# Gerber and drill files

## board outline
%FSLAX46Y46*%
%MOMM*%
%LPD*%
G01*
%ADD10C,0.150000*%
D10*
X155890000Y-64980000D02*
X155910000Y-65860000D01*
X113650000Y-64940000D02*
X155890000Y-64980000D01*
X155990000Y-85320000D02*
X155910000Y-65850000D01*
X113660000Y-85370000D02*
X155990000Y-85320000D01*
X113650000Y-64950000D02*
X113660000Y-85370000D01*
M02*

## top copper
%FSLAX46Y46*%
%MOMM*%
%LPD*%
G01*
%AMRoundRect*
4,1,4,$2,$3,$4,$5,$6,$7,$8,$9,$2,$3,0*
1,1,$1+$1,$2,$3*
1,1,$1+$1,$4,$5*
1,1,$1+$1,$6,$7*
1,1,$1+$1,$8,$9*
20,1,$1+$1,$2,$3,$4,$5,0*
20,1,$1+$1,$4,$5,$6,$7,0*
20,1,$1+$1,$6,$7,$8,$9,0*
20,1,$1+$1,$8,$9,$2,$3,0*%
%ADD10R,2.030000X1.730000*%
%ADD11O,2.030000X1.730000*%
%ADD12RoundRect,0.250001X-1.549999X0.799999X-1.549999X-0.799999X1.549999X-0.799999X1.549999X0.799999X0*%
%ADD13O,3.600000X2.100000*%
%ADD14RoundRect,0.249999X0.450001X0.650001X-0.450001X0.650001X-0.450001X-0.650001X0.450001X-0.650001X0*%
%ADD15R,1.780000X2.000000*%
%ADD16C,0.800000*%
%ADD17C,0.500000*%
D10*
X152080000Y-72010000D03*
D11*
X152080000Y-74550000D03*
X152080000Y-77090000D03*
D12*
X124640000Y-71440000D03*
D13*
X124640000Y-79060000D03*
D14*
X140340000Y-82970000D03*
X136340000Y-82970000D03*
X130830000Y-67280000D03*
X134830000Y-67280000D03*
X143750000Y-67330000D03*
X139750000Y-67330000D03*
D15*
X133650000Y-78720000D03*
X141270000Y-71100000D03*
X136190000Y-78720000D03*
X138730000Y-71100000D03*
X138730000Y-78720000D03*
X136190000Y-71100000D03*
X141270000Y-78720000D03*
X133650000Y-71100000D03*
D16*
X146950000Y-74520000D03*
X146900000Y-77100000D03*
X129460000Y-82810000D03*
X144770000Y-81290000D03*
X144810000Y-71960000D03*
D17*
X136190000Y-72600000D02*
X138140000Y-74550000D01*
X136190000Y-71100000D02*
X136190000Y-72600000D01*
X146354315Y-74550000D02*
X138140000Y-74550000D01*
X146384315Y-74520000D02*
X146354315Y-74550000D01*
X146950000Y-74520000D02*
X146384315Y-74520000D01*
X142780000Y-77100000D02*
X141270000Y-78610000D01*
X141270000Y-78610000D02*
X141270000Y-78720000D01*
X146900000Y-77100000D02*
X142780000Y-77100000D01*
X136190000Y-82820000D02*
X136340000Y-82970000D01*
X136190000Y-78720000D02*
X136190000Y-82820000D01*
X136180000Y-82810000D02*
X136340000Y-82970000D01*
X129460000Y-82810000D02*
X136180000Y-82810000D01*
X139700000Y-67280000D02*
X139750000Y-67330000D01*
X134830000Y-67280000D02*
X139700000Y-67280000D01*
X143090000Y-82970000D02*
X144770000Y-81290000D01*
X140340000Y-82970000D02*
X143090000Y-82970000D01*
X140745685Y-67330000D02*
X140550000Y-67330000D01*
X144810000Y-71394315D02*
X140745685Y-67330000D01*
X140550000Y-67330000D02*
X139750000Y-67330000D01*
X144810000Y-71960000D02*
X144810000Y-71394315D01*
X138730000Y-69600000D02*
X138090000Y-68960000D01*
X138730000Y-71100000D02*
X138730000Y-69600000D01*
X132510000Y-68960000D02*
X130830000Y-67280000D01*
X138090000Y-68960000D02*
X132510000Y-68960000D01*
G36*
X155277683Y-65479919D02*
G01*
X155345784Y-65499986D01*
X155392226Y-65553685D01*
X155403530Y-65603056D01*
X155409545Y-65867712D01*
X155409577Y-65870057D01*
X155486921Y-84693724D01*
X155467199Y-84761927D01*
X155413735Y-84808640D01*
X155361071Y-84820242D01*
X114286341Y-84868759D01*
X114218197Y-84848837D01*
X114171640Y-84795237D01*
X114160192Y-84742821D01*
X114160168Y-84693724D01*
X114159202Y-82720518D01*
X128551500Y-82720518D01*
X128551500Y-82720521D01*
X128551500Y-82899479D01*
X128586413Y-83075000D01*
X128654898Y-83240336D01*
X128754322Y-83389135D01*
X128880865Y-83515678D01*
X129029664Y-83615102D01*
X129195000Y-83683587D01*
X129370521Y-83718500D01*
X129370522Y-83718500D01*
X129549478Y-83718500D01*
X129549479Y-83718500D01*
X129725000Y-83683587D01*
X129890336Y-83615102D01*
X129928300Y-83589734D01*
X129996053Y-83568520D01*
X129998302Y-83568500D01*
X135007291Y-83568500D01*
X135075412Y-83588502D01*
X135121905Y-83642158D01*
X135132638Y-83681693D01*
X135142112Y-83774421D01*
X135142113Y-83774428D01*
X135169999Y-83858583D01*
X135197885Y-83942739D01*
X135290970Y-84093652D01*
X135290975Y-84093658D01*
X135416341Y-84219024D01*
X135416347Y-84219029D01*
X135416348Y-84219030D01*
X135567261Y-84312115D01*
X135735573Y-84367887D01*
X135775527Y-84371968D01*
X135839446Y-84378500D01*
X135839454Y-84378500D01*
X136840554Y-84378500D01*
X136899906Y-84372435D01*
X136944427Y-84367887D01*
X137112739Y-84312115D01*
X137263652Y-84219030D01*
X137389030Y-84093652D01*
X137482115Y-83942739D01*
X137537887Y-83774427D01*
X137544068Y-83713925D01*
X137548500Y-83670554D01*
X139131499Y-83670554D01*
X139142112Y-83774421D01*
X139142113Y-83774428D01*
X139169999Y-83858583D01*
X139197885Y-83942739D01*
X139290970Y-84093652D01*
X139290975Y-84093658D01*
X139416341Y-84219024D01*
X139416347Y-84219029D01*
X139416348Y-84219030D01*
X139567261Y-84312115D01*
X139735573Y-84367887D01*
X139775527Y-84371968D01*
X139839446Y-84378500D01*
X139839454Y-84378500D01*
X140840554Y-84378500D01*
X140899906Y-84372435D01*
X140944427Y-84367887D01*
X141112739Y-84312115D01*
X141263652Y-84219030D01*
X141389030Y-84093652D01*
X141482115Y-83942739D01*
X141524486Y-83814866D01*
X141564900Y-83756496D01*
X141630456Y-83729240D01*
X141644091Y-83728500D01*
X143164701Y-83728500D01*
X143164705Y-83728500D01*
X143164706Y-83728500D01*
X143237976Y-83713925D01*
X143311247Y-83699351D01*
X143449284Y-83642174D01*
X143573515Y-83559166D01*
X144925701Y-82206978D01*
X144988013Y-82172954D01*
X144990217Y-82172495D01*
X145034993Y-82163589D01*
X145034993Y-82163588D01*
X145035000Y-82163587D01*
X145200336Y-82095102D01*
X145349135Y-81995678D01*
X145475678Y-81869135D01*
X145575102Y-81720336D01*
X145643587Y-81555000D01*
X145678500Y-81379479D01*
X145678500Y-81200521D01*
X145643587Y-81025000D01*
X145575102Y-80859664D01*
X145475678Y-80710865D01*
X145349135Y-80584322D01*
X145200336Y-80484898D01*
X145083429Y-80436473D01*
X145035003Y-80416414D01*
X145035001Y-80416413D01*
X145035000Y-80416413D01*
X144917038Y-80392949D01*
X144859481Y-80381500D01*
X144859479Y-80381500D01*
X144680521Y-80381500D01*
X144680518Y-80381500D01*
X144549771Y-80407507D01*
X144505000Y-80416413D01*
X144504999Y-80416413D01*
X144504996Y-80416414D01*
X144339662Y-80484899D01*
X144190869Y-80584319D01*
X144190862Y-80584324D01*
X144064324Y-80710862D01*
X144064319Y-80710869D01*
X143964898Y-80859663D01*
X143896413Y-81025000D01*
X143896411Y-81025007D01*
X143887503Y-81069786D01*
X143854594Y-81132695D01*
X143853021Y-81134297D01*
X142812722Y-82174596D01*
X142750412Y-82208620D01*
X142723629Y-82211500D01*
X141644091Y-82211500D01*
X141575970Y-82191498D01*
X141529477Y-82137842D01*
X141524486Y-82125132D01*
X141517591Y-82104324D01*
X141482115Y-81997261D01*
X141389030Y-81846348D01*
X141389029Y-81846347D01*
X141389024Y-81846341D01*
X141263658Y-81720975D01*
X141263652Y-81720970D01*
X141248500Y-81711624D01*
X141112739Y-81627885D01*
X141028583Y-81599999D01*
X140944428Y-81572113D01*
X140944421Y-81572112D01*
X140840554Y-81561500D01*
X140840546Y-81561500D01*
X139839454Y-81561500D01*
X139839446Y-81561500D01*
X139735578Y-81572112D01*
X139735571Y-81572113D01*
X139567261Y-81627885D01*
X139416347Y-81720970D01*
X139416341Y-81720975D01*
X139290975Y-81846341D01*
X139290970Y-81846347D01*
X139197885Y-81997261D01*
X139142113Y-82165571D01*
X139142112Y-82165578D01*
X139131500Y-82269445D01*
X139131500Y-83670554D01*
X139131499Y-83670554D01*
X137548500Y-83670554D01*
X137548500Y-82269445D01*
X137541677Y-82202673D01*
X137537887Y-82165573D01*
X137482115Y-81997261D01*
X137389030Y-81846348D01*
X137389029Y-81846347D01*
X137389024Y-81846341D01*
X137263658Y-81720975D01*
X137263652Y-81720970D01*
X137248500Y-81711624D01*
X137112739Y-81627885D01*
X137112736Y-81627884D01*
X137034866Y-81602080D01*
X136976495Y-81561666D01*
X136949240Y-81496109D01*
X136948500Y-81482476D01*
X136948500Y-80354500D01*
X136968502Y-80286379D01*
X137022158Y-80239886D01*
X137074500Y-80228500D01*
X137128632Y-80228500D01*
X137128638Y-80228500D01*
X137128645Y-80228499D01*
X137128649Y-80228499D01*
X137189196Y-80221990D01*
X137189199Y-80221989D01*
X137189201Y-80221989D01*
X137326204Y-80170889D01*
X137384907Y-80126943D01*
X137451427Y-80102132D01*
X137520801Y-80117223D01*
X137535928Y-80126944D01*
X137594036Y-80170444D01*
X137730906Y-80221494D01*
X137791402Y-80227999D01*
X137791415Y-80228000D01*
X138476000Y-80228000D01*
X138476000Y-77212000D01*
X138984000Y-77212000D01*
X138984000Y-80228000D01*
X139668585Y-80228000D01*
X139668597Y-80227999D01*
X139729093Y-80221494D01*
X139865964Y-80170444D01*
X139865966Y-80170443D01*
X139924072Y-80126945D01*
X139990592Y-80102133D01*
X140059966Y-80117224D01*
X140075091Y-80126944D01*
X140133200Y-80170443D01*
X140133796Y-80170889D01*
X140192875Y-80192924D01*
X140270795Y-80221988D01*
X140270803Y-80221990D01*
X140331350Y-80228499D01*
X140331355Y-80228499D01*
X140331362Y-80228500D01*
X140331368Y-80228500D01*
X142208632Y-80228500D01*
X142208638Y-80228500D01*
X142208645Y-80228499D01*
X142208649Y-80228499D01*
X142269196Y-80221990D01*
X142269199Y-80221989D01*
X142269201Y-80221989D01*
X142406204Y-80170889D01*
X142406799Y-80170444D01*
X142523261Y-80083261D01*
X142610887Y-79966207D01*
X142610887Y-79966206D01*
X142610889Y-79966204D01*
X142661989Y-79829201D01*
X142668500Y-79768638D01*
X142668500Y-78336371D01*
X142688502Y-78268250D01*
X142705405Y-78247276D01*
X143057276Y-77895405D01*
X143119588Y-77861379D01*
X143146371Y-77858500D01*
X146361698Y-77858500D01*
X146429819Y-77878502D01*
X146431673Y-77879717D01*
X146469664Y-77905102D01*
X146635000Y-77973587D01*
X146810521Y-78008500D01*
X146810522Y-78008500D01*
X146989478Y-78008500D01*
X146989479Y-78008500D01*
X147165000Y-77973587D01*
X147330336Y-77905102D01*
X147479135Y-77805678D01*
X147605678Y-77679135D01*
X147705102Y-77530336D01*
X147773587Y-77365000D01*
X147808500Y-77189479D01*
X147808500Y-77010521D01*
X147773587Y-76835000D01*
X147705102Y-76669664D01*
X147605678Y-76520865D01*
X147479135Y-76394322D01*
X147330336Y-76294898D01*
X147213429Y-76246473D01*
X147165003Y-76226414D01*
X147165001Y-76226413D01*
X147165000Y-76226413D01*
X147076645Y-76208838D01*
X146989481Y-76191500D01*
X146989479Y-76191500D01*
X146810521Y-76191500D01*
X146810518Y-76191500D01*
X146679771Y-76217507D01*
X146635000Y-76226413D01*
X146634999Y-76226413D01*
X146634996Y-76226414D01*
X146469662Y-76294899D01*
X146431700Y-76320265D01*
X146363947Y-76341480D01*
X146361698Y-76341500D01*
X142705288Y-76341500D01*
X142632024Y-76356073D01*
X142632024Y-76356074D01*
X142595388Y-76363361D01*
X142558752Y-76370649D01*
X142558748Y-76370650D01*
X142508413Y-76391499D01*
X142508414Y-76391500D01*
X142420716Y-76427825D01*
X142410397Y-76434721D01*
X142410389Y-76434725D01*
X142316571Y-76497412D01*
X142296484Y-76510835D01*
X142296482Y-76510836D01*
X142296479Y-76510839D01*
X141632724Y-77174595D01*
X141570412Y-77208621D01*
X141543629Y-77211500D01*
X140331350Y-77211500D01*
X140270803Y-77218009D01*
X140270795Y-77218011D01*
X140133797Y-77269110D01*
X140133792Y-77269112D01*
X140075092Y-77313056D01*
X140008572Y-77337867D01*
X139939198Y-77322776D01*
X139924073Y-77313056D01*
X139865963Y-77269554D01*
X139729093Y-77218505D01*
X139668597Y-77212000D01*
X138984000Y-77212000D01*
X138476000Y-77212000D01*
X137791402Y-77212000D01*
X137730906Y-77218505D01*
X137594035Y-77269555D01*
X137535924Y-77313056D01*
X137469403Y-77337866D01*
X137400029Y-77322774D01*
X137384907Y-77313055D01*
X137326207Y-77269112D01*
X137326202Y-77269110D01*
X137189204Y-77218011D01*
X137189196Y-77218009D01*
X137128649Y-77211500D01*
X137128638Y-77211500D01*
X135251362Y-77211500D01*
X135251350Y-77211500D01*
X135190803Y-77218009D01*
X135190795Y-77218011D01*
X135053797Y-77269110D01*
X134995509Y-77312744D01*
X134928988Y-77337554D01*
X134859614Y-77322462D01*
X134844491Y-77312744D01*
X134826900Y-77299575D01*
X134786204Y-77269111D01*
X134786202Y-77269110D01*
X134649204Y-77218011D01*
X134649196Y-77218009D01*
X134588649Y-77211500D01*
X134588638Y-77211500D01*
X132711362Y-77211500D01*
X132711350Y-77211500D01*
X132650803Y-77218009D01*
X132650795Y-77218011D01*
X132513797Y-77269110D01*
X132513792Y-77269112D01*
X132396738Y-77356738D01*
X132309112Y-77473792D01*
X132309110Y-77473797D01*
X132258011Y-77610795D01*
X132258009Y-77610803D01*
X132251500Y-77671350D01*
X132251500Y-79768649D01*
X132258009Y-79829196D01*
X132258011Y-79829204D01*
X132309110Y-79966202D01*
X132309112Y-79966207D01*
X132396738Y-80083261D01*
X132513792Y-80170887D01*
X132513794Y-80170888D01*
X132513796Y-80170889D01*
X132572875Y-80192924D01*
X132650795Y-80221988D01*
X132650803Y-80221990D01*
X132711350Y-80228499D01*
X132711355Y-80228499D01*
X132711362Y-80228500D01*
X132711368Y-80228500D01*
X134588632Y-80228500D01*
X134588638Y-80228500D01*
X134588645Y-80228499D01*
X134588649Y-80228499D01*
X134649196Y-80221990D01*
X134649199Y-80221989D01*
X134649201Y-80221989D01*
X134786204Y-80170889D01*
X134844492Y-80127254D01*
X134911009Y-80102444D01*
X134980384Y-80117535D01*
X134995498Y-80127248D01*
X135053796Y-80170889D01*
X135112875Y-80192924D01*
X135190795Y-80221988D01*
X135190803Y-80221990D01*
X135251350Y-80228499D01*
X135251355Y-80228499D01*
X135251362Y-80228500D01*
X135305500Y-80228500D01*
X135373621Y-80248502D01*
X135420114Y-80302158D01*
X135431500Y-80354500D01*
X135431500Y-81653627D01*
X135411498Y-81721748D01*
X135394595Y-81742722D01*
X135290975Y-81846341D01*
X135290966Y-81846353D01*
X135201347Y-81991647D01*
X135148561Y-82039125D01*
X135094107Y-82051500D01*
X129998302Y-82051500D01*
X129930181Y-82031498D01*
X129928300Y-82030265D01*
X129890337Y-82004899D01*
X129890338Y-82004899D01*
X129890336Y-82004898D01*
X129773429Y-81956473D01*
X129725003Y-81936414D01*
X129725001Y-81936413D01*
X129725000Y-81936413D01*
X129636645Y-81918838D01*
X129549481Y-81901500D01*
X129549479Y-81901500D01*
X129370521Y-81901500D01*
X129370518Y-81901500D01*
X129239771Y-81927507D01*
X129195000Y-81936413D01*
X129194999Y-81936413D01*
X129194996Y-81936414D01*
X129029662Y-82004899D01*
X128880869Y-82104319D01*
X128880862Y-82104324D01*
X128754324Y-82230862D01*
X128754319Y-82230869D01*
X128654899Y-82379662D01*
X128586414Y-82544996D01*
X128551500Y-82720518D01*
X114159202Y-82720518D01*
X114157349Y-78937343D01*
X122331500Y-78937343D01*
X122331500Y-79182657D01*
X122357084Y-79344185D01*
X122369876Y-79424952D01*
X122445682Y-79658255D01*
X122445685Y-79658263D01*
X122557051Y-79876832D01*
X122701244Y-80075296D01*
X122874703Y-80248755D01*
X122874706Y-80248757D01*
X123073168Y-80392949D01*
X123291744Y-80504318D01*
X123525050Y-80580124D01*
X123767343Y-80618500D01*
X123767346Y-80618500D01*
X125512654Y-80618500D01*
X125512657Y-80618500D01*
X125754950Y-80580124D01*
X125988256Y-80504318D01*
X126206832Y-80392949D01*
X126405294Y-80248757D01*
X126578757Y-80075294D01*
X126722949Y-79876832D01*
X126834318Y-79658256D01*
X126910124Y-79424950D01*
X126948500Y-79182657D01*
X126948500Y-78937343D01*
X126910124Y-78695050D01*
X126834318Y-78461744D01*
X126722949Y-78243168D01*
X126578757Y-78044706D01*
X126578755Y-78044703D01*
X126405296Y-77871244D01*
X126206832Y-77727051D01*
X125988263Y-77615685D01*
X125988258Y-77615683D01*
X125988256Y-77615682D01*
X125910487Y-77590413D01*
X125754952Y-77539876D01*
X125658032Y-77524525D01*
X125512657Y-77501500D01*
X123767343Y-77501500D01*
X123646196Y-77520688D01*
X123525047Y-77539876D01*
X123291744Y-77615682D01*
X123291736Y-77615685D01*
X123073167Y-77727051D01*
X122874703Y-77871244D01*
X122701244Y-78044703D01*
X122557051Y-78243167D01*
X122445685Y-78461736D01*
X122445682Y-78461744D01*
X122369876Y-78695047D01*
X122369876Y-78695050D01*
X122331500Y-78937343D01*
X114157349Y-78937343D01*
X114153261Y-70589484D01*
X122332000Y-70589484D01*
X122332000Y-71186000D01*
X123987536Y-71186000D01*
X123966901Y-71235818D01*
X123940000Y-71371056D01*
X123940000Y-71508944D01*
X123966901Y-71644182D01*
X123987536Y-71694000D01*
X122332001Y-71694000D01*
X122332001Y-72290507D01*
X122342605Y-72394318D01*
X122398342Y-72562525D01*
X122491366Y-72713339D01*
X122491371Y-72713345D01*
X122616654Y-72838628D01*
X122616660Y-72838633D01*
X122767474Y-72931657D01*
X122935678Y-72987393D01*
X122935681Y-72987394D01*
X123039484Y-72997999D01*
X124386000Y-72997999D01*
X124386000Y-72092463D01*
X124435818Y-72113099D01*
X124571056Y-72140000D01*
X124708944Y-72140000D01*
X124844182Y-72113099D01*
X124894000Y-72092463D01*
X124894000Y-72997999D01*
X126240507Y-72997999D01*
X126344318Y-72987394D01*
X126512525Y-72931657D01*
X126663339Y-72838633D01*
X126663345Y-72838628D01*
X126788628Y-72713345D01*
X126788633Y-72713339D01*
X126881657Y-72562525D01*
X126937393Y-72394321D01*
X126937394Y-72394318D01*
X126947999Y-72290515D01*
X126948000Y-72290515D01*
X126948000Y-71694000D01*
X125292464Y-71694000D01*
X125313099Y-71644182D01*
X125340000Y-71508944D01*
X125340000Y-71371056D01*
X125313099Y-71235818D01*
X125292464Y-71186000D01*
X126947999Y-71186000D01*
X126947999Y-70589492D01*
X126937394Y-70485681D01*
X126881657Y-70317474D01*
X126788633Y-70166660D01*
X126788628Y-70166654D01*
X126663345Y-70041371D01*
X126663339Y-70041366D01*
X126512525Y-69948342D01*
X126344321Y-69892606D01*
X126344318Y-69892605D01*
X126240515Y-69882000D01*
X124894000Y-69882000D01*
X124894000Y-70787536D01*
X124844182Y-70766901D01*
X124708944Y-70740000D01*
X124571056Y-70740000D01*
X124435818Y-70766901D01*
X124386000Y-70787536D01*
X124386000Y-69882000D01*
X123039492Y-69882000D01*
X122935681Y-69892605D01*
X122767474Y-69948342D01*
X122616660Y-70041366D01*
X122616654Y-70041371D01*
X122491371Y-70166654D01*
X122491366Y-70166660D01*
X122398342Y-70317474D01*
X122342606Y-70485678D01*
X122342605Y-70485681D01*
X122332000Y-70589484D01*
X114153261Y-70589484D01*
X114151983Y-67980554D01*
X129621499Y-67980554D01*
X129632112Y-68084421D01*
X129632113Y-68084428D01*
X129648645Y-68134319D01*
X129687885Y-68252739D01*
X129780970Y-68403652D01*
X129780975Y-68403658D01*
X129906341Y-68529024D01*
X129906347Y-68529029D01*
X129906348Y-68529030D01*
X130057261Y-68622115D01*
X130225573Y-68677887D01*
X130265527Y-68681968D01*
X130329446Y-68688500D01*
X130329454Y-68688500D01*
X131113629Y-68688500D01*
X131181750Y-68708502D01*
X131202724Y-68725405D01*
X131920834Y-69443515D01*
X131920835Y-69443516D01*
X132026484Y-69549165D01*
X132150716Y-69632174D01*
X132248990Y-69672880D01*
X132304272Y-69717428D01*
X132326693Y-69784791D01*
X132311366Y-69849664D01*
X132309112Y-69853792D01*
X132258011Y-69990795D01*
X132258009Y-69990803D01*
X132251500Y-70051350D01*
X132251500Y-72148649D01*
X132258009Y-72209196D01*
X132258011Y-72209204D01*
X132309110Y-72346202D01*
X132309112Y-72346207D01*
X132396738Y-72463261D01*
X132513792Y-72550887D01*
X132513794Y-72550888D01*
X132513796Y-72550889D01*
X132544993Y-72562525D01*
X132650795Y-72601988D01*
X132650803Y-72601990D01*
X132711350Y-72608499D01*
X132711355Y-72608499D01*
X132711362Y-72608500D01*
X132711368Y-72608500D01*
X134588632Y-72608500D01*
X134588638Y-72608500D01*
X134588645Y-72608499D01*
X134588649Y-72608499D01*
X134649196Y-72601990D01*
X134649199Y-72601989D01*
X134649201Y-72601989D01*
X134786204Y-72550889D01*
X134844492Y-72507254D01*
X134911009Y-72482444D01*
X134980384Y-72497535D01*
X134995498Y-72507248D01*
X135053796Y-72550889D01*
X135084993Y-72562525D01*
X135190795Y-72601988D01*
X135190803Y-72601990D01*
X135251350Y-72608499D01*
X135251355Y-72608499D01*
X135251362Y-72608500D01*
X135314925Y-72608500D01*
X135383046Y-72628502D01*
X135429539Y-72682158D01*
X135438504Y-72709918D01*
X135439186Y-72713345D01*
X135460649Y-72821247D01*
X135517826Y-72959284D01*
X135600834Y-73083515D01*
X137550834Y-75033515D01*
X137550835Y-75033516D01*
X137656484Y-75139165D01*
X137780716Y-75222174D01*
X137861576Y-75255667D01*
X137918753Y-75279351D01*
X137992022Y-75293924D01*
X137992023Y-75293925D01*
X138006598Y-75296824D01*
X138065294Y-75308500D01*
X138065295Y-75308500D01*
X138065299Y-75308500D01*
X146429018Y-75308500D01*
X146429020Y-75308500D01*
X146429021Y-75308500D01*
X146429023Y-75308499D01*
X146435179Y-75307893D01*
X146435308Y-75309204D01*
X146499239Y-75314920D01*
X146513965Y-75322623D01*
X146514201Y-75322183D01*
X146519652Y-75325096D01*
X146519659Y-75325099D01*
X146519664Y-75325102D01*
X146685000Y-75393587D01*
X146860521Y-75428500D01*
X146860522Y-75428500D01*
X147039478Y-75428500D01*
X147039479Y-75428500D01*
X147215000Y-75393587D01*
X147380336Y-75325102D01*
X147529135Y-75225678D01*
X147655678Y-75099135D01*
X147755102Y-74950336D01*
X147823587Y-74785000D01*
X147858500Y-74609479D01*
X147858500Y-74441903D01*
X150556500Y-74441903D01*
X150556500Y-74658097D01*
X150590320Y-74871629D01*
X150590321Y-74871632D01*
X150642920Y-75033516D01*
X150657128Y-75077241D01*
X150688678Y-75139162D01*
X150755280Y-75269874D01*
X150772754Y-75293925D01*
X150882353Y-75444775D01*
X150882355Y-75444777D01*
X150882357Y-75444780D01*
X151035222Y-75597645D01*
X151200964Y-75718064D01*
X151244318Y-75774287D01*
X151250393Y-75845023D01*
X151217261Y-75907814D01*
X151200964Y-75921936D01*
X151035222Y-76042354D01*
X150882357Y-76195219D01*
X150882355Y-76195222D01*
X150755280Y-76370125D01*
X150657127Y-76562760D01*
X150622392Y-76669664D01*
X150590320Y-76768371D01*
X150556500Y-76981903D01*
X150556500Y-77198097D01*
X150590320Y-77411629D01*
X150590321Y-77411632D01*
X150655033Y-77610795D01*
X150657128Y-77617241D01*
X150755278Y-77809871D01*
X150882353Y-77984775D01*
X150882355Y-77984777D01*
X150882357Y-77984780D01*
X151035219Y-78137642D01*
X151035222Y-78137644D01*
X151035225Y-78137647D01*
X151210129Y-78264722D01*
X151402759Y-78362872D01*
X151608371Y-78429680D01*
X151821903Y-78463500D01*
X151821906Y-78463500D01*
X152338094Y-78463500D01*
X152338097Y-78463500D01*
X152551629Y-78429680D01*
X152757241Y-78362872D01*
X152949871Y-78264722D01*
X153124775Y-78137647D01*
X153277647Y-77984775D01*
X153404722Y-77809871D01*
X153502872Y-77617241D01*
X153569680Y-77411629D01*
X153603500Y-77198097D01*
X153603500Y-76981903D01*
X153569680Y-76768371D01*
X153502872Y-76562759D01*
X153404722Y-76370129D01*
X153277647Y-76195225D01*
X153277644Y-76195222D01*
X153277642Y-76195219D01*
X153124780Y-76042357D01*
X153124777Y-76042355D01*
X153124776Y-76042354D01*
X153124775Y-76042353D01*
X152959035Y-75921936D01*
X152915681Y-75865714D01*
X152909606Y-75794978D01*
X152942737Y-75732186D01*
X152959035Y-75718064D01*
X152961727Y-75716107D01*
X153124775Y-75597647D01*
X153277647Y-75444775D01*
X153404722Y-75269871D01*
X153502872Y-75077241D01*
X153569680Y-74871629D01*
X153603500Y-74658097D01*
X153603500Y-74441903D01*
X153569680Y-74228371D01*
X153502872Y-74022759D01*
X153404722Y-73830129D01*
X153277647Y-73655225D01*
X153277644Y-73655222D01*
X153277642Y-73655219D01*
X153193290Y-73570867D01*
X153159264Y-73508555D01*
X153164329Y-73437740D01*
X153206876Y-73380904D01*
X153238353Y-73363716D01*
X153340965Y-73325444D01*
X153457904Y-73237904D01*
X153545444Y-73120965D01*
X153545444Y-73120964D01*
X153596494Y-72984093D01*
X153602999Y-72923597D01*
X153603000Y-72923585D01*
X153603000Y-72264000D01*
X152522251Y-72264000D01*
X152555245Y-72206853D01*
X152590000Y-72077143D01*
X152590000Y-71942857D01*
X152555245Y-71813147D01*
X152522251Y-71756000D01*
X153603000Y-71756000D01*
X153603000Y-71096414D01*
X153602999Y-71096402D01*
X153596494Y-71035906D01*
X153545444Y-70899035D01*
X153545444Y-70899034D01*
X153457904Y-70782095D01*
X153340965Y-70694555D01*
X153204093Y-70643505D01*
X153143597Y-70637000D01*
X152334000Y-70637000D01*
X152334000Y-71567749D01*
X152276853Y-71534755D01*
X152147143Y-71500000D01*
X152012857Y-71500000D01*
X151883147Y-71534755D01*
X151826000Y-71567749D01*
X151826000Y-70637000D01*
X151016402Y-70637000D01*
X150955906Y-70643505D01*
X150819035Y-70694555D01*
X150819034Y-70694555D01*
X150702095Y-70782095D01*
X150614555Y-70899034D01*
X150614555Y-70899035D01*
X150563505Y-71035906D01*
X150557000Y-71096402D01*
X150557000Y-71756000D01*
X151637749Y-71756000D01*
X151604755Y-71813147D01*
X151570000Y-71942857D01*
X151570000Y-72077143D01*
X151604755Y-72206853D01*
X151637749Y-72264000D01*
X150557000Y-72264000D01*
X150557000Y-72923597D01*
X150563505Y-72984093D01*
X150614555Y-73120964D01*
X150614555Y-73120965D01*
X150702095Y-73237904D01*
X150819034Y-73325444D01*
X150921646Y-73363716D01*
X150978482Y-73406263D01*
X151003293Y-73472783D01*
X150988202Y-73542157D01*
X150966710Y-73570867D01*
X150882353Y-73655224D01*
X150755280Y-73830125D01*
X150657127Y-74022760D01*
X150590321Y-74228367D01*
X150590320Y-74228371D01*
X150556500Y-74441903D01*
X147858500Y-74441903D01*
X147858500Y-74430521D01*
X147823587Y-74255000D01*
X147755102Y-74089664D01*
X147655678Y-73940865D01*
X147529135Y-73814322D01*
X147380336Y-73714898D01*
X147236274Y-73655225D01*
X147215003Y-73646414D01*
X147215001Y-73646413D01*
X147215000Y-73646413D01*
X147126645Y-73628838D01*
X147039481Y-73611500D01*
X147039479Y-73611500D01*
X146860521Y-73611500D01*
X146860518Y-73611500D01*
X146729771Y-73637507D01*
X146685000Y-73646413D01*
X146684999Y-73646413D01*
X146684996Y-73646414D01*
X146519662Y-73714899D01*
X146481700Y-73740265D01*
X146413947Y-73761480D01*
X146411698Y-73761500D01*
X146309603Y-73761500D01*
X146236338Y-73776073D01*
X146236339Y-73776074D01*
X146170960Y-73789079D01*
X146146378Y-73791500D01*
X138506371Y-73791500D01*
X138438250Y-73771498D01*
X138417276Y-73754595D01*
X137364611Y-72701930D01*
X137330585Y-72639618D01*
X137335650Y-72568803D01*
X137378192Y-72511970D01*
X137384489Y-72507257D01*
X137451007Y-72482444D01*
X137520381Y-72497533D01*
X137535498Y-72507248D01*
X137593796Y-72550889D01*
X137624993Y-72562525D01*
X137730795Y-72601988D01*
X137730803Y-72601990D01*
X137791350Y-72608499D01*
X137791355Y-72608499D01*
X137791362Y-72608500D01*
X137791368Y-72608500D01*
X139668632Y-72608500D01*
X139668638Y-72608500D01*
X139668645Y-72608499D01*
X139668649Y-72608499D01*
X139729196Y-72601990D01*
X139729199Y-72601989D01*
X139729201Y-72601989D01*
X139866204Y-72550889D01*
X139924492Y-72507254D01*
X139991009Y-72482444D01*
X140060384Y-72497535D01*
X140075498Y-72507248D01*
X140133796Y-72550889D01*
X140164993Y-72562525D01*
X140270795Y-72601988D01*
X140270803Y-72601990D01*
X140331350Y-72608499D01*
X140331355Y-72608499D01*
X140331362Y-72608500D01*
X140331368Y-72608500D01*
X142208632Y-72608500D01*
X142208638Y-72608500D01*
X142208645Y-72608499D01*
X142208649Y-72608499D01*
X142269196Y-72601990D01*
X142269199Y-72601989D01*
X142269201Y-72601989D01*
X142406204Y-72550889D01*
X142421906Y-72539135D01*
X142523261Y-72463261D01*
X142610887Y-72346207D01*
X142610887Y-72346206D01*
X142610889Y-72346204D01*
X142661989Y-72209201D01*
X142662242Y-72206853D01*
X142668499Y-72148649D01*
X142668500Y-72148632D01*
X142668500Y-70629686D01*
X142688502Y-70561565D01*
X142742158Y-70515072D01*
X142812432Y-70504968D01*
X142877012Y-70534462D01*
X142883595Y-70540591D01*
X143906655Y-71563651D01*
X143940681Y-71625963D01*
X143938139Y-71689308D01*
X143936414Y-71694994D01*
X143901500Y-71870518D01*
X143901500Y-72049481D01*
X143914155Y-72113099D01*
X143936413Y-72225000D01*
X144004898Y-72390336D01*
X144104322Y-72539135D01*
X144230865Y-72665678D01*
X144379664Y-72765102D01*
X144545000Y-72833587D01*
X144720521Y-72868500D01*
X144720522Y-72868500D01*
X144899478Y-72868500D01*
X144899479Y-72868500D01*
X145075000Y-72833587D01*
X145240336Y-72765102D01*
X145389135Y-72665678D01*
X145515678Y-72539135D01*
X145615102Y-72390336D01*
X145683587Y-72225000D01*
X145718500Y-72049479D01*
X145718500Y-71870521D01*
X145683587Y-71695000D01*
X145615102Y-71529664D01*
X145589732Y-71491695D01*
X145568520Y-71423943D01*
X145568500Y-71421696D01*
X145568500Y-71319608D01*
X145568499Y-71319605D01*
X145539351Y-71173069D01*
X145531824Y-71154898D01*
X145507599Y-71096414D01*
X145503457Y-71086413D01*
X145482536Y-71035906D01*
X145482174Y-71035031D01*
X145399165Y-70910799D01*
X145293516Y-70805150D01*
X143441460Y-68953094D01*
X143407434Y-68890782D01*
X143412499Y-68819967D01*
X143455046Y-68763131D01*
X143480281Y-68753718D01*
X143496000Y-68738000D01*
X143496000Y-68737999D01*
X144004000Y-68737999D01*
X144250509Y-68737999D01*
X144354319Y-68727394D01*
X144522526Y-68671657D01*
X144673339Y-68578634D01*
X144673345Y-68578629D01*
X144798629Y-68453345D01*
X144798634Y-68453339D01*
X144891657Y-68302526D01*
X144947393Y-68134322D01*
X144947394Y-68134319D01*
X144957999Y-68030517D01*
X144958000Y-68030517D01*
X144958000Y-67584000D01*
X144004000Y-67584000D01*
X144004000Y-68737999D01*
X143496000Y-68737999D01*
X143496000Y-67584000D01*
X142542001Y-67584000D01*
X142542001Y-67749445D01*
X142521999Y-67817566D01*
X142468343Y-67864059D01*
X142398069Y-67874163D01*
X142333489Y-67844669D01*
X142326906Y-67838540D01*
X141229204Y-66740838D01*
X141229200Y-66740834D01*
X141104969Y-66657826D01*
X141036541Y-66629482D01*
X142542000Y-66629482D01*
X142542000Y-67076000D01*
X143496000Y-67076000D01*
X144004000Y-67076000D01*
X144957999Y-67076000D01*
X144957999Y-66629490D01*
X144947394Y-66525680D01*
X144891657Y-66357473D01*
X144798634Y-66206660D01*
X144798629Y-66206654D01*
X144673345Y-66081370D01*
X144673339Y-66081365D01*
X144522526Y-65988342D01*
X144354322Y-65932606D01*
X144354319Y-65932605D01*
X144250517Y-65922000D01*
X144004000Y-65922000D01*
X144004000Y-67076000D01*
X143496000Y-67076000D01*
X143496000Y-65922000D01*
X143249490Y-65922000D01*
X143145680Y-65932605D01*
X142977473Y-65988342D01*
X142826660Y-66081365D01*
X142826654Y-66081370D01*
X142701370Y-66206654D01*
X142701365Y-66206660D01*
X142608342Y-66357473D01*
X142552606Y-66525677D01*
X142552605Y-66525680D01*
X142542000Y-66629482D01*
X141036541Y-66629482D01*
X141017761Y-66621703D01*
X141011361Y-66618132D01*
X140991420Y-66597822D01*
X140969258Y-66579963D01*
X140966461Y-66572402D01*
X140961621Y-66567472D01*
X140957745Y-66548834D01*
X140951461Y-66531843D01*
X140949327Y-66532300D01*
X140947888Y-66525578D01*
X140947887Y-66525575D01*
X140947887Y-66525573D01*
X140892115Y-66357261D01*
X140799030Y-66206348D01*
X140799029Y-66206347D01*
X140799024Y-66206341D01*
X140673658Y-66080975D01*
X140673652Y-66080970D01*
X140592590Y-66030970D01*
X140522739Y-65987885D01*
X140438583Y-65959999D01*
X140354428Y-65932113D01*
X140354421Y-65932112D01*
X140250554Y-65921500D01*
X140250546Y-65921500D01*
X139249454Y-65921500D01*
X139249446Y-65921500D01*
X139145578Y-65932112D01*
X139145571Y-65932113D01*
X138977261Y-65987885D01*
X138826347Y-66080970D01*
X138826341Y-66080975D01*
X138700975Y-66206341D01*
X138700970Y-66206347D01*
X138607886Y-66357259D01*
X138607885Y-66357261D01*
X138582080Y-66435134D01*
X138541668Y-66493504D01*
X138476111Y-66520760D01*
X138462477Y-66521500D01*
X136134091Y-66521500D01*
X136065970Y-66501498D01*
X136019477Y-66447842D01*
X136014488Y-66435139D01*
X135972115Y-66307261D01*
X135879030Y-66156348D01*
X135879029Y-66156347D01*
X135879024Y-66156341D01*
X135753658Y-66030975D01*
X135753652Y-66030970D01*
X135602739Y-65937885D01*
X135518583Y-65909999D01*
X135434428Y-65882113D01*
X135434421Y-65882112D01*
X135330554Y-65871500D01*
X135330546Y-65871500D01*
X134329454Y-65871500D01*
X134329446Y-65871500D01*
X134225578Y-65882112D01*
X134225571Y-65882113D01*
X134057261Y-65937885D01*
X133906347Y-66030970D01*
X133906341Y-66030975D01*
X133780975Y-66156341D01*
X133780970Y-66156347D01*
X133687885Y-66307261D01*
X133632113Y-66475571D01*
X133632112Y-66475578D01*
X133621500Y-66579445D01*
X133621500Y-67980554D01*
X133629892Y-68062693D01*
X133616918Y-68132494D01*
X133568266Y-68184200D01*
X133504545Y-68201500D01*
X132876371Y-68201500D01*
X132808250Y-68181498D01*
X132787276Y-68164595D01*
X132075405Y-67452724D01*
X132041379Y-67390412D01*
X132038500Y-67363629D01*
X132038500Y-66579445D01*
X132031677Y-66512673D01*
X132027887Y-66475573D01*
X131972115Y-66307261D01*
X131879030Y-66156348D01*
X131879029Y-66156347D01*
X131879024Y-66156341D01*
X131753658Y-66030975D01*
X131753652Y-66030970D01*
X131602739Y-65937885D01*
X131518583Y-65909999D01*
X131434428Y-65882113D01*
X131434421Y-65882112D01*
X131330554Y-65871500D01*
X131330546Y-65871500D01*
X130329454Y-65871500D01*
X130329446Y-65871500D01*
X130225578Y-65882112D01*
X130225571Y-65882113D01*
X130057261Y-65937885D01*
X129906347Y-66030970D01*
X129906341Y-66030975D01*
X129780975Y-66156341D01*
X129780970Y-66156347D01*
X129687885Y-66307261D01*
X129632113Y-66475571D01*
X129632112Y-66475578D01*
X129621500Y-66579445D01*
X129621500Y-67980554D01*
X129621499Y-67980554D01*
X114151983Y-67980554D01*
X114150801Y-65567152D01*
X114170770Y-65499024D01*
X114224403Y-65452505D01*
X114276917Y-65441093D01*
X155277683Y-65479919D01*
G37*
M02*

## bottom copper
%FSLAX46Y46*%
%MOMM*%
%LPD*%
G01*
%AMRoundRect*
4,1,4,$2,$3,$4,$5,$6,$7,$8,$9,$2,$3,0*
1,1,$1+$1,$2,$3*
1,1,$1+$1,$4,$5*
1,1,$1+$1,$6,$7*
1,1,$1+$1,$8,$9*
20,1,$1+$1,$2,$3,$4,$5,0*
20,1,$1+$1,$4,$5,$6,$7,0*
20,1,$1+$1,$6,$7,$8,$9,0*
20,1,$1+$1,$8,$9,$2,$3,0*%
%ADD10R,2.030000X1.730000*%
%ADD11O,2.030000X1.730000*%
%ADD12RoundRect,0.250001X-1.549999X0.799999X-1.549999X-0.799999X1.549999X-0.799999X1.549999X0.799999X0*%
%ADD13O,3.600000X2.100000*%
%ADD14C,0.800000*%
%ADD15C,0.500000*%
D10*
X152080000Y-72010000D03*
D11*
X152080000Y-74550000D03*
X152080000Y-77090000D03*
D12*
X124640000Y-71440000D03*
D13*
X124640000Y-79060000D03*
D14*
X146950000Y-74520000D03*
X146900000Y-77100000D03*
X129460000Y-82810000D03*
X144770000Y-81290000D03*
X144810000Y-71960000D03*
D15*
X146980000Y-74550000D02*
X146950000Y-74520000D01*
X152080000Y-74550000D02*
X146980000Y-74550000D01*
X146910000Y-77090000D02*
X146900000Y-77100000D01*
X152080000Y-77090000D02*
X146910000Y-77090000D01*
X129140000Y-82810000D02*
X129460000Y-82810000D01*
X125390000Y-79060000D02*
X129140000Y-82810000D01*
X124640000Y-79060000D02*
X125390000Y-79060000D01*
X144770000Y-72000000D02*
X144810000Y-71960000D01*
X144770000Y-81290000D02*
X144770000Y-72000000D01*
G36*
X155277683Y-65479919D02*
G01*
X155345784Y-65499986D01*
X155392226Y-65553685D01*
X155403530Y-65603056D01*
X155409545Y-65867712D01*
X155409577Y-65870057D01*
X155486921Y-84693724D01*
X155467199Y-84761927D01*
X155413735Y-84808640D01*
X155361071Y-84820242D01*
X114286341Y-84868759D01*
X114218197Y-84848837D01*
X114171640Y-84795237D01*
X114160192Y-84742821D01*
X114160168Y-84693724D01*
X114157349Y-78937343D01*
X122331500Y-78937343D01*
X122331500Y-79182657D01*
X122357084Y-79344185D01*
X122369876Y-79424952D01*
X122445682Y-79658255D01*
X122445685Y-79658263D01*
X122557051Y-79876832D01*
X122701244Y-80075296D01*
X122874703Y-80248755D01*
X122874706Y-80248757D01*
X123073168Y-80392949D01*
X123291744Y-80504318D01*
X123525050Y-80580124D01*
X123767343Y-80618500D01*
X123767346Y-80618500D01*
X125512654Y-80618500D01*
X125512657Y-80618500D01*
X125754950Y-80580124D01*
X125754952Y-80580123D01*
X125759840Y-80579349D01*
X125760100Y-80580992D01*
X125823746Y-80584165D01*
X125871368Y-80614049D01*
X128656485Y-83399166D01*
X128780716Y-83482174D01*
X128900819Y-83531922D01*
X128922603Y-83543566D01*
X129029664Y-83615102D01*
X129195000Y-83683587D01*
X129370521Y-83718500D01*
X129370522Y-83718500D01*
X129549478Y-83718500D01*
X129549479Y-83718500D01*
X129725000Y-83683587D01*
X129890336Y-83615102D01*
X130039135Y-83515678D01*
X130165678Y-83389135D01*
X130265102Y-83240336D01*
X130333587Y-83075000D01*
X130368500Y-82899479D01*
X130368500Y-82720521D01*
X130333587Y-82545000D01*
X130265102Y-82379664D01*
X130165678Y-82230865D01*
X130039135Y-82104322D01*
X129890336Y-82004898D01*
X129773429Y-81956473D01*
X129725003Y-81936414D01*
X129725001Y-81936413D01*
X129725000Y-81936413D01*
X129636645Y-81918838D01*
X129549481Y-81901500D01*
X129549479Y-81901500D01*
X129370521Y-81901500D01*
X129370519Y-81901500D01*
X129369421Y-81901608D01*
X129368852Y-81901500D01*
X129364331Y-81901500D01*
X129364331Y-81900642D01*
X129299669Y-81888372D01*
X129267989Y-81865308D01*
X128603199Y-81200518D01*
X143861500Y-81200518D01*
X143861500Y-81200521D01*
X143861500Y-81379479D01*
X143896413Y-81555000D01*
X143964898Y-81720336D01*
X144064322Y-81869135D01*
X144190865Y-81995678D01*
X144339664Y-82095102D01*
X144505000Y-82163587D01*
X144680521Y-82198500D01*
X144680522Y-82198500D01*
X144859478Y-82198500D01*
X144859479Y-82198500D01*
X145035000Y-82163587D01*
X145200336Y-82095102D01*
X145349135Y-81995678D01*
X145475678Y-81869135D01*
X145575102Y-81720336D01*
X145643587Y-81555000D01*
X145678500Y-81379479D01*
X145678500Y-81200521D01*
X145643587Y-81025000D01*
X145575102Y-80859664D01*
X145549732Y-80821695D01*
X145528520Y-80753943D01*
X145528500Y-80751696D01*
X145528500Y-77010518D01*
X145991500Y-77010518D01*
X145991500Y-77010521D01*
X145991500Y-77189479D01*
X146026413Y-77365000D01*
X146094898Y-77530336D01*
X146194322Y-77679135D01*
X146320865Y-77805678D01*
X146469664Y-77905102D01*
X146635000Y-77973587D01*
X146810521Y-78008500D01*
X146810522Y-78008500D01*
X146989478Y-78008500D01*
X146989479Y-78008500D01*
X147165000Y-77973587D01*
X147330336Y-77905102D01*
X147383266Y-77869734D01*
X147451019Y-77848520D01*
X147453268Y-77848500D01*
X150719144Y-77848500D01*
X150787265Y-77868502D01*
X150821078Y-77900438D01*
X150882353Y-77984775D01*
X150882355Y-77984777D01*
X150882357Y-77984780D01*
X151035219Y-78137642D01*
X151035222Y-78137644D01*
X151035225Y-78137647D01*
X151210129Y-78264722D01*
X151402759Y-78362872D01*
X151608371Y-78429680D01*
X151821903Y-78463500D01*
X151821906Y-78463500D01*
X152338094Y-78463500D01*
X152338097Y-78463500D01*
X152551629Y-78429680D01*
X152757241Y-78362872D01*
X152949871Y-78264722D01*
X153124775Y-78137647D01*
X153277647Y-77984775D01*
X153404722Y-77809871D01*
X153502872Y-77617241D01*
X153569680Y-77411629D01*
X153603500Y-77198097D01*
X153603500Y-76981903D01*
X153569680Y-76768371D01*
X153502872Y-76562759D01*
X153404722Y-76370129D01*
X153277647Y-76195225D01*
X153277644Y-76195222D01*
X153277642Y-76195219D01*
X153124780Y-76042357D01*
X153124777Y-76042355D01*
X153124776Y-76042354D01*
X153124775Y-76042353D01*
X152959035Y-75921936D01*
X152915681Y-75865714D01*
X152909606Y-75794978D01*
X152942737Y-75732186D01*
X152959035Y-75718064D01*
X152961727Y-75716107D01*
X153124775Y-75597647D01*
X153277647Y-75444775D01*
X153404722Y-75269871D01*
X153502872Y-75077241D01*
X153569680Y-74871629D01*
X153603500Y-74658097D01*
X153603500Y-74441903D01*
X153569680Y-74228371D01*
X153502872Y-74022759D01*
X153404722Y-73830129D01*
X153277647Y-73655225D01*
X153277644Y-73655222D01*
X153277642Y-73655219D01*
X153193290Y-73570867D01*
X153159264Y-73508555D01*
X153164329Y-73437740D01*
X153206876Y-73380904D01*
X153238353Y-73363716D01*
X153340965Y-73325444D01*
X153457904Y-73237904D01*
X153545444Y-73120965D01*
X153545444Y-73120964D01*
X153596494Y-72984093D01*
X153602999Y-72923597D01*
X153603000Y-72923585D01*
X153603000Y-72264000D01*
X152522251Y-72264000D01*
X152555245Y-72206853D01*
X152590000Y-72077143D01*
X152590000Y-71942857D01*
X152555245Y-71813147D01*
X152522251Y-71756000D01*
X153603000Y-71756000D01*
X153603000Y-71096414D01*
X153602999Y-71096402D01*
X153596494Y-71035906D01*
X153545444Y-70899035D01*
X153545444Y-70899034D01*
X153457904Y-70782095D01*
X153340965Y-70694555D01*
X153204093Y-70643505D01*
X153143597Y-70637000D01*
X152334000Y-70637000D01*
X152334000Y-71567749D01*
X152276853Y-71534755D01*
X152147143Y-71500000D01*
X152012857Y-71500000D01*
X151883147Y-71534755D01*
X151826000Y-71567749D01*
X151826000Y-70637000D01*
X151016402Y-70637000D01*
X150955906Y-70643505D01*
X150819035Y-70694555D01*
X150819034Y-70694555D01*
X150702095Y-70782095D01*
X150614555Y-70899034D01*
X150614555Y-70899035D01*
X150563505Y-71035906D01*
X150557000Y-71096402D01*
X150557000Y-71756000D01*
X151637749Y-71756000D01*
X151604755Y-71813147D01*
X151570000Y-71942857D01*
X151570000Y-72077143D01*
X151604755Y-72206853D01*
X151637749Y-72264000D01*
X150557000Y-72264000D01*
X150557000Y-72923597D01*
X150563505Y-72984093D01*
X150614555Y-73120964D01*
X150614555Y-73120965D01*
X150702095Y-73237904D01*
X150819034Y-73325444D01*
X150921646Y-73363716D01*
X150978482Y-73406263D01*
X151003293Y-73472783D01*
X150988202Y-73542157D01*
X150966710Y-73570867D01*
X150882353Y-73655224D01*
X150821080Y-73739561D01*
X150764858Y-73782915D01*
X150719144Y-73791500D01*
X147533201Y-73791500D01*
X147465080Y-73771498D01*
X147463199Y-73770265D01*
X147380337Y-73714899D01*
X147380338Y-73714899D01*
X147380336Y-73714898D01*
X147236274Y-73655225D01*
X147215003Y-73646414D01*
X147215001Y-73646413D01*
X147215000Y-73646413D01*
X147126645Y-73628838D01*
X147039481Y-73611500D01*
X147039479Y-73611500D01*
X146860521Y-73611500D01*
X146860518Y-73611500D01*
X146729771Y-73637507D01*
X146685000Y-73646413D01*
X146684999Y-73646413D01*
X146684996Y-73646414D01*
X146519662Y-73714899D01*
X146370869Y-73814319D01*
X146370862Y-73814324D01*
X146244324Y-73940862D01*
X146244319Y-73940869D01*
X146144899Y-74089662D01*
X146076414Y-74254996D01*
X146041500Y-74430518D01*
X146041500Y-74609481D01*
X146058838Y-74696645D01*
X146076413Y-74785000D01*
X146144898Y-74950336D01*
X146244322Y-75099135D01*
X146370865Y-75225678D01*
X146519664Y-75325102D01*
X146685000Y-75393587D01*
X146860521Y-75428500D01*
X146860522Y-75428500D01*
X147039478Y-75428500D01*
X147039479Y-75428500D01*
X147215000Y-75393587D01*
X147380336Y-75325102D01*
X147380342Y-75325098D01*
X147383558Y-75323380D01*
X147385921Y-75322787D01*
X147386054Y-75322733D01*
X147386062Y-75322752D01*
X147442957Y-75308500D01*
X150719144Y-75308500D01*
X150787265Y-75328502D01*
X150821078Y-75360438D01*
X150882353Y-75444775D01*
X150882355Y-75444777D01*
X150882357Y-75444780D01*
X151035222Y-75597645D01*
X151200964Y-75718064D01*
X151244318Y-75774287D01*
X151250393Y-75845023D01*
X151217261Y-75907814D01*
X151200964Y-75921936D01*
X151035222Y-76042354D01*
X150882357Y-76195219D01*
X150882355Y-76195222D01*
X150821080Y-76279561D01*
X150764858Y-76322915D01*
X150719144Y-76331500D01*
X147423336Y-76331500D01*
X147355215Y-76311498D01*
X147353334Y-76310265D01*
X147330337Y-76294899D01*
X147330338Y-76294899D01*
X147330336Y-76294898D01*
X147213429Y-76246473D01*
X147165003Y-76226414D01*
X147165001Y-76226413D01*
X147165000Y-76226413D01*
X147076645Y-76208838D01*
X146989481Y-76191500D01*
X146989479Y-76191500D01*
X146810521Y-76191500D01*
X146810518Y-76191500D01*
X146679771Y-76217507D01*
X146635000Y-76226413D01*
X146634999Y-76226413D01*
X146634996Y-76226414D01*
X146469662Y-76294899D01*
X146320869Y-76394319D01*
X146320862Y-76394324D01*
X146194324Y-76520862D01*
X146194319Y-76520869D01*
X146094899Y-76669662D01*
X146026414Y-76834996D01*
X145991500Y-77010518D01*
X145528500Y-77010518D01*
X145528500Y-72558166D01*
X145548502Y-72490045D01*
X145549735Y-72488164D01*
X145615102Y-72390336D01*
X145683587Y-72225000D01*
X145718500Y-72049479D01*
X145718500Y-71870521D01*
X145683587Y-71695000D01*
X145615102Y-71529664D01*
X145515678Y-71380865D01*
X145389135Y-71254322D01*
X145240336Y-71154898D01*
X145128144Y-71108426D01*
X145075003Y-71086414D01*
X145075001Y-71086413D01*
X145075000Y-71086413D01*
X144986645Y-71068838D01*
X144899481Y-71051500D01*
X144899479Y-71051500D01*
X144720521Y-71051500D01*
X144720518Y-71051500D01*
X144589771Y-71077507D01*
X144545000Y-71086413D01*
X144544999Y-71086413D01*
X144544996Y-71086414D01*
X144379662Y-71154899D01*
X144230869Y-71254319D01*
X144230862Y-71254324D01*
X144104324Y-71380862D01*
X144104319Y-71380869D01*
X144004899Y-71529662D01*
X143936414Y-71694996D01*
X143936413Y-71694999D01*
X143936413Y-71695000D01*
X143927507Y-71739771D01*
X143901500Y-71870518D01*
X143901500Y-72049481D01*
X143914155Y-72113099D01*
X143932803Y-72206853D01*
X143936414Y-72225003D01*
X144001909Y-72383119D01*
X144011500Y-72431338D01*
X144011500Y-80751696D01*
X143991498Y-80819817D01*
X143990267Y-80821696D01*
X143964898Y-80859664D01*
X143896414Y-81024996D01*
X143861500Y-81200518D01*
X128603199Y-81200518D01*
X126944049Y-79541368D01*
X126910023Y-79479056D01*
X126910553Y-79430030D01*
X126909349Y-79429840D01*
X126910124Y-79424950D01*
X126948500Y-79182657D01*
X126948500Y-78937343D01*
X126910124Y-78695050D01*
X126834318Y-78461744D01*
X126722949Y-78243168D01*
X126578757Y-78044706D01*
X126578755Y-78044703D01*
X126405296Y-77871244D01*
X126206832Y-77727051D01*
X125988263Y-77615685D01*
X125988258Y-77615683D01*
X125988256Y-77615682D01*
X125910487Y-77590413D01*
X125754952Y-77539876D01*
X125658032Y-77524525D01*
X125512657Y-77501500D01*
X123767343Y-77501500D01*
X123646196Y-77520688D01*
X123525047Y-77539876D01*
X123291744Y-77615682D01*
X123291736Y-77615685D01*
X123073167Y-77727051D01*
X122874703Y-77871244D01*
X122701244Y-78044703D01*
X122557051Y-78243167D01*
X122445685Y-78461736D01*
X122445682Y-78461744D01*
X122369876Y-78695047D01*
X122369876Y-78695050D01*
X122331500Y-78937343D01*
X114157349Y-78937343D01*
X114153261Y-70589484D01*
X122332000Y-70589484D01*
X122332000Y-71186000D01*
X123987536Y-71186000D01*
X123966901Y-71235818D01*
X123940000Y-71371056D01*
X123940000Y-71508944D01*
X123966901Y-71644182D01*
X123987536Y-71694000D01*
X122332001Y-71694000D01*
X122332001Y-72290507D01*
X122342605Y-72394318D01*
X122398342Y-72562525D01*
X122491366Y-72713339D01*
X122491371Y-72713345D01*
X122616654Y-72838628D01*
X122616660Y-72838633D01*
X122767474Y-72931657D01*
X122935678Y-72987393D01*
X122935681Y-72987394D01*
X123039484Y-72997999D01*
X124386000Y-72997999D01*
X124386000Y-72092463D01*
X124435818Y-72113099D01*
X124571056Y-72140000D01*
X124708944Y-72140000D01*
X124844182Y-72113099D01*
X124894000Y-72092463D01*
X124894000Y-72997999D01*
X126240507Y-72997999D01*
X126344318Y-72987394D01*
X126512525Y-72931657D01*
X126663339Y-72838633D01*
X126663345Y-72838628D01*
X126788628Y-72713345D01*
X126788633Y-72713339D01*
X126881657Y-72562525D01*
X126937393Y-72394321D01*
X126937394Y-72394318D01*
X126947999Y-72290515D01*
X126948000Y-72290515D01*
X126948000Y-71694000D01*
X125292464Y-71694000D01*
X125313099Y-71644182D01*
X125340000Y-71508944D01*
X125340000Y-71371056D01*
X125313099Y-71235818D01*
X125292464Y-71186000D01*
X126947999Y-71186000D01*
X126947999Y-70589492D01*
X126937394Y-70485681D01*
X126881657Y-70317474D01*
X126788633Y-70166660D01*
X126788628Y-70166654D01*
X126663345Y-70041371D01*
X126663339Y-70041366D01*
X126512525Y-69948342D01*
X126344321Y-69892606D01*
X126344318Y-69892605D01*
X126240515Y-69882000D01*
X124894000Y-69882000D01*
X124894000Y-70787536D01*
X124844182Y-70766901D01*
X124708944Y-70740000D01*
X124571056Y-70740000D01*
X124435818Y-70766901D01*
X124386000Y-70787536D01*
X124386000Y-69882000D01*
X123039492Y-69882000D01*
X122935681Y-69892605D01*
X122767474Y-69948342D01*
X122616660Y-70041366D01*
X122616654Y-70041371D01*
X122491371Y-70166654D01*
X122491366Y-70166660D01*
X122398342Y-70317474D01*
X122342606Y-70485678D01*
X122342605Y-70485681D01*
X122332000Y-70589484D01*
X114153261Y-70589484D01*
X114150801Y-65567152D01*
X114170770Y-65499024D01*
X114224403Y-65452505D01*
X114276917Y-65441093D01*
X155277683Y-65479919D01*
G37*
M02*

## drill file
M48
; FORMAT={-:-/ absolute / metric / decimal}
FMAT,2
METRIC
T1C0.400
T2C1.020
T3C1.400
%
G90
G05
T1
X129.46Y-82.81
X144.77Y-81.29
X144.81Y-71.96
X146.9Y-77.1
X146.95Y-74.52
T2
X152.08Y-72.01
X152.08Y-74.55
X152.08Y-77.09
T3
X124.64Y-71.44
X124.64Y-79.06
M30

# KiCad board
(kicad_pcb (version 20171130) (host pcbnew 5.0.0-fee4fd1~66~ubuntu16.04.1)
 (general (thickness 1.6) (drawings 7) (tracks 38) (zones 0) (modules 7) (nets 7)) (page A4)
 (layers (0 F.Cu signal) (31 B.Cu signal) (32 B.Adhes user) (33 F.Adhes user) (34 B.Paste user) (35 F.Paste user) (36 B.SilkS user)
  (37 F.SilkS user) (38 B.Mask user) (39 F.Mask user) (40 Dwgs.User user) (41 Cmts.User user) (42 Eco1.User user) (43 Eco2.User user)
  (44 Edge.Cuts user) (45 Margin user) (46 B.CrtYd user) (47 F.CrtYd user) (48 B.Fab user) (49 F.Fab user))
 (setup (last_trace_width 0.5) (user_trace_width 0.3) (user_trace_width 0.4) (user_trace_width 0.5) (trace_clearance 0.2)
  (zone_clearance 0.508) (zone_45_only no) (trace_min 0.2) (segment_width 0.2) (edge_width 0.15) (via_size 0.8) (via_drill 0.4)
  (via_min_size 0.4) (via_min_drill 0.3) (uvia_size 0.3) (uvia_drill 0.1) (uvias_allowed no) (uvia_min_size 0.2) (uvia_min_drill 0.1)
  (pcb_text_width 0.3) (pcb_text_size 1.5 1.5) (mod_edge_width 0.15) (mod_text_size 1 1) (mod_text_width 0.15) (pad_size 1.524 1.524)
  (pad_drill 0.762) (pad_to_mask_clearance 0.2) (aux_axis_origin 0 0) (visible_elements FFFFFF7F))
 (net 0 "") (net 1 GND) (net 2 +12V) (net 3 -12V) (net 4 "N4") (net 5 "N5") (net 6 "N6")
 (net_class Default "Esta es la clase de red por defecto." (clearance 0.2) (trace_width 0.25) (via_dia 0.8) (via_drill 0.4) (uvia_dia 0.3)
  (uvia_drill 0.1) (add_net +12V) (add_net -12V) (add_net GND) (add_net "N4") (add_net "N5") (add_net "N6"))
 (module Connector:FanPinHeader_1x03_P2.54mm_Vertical (layer F.Cu) (at 152.08 72.01 270)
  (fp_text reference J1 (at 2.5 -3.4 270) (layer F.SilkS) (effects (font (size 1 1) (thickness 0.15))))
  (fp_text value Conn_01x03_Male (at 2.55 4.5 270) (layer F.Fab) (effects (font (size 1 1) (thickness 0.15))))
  (pad 1 thru_hole rect (at 0 0) (size 2.03 1.73) (drill 1.02) (layers *.Cu *.Mask) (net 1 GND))
  (pad 2 thru_hole oval (at 2.54 0) (size 2.03 1.73) (drill 1.02) (layers *.Cu *.Mask) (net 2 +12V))
  (pad 3 thru_hole oval (at 5.08 0) (size 2.03 1.73) (drill 1.02) (layers *.Cu *.Mask) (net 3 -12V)))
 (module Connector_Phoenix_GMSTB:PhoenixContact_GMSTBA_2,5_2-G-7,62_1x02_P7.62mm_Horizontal (layer F.Cu) (at 124.64 71.44 270)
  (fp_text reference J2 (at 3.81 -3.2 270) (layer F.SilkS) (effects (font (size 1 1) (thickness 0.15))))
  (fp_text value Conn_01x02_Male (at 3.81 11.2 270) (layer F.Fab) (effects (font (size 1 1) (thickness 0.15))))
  (pad 1 thru_hole roundrect (at 0 0 270) (size 2.1 3.6) (drill 1.4) (layers *.Cu *.Mask) (roundrect_rratio 0.119048) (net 1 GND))
  (pad 2 thru_hole oval (at 7.62 0 270) (size 2.1 3.6) (drill 1.4) (layers *.Cu *.Mask) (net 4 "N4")))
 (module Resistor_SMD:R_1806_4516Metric (layer F.Cu) (at 138.34 82.97 180)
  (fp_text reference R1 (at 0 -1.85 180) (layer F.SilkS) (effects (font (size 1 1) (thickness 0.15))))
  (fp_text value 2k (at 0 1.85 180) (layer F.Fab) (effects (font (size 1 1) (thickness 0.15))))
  (pad 1 smd roundrect (at -2 0 180) (size 1.4 1.8) (layers F.Cu F.Paste F.Mask) (roundrect_rratio 0.178571) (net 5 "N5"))
  (pad 2 smd roundrect (at 2 0 180) (size 1.4 1.8) (layers F.Cu F.Paste F.Mask) (roundrect_rratio 0.178571) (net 4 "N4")))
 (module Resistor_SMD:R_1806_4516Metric (layer F.Cu) (at 132.83 67.28 180)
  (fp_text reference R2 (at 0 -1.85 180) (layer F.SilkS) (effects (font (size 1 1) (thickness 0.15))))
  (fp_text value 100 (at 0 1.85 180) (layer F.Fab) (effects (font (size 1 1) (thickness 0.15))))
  (pad 2 smd roundrect (at 2 0 180) (size 1.4 1.8) (layers F.Cu F.Paste F.Mask) (roundrect_rratio 0.178571) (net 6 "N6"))
  (pad 1 smd roundrect (at -2 0 180) (size 1.4 1.8) (layers F.Cu F.Paste F.Mask) (roundrect_rratio 0.178571) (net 5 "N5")))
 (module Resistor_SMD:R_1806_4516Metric (layer F.Cu) (at 141.75 67.33 180)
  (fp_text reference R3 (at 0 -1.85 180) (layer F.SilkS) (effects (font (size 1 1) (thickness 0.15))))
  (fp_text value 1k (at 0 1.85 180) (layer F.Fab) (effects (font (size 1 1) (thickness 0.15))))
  (pad 1 smd roundrect (at -2 0 180) (size 1.4 1.8) (layers F.Cu F.Paste F.Mask) (roundrect_rratio 0.178571) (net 1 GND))
  (pad 2 smd roundrect (at 2 0 180) (size 1.4 1.8) (layers F.Cu F.Paste F.Mask) (roundrect_rratio 0.178571) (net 5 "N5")))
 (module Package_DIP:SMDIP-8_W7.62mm (layer F.Cu) (at 137.46 74.91 90)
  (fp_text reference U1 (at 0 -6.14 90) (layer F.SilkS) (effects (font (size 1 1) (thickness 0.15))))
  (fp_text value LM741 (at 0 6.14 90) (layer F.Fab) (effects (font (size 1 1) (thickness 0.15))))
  (pad 1 smd rect (at -3.81 -3.81 90) (size 2 1.78) (layers F.Cu F.Paste F.Mask))
  (pad 5 smd rect (at 3.81 3.81 90) (size 2 1.78) (layers F.Cu F.Paste F.Mask))
  (pad 2 smd rect (at -3.81 -1.27 90) (size 2 1.78) (layers F.Cu F.Paste F.Mask) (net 4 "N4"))
  (pad 6 smd rect (at 3.81 1.27 90) (size 2 1.78) (layers F.Cu F.Paste F.Mask) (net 6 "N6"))
  (pad 3 smd rect (at -3.81 1.27 90) (size 2 1.78) (layers F.Cu F.Paste F.Mask) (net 1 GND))
  (pad 7 smd rect (at 3.81 -1.27 90) (size 2 1.78) (layers F.Cu F.Paste F.Mask) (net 2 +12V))
  (pad 4 smd rect (at -3.81 3.81 90) (size 2 1.78) (layers F.Cu F.Paste F.Mask) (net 3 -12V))
  (pad 8 smd rect (at 3.81 -3.81 90) (size 2 1.78) (layers F.Cu F.Paste F.Mask)))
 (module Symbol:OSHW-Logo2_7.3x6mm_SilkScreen (layer F.Cu) (at 152.07 82.09)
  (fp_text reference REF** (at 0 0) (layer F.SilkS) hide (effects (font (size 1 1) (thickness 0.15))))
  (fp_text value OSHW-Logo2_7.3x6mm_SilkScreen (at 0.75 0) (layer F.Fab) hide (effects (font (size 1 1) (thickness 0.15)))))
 (gr_line (start 155.89 64.98) (end 155.91 65.86) (layer Edge.Cuts) (width 0.15))
 (gr_line (start 113.65 64.94) (end 155.89 64.98) (layer Edge.Cuts) (width 0.15))
 (gr_line (start 155.99 85.32) (end 155.91 65.85) (layer Edge.Cuts) (width 0.15))
 (gr_line (start 113.66 85.37) (end 155.99 85.32) (layer Edge.Cuts) (width 0.15))
 (gr_line (start 113.65 64.95) (end 113.66 85.37) (layer Edge.Cuts) (width 0.15))
 (segment (start 136.19 72.6) (end 138.14 74.55) (width 0.5) (layer F.Cu) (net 2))
 (segment (start 136.19 71.1) (end 136.19 72.6) (width 0.5) (layer F.Cu) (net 2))
 (segment (start 146.98 74.55) (end 146.95 74.52) (width 0.5) (layer B.Cu) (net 2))
 (via (at 146.95 74.52) (size 0.8) (drill 0.4) (layers F.Cu B.Cu) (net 2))
 (segment (start 152.08 74.55) (end 146.98 74.55) (width 0.5) (layer B.Cu) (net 2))
 (segment (start 146.354315 74.55) (end 138.14 74.55) (width 0.5) (layer F.Cu) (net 2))
 (segment (start 146.384315 74.52) (end 146.354315 74.55) (width 0.5) (layer F.Cu) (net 2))
 (segment (start 146.95 74.52) (end 146.384315 74.52) (width 0.5) (layer F.Cu) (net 2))
 (via (at 146.9 77.1) (size 0.8) (drill 0.4) (layers F.Cu B.Cu) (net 3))
 (segment (start 146.91 77.09) (end 146.9 77.1) (width 0.5) (layer B.Cu) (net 3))
 (segment (start 152.08 77.09) (end 146.91 77.09) (width 0.5) (layer B.Cu) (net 3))
 (segment (start 142.78 77.1) (end 141.27 78.61) (width 0.5) (layer F.Cu) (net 3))
 (segment (start 141.27 78.61) (end 141.27 78.72) (width 0.5) (layer F.Cu) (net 3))
 (segment (start 146.9 77.1) (end 142.78 77.1) (width 0.5) (layer F.Cu) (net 3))
 (segment (start 136.19 82.82) (end 136.34 82.97) (width 0.5) (layer F.Cu) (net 4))
 (segment (start 136.19 78.72) (end 136.19 82.82) (width 0.5) (layer F.Cu) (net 4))
 (segment (start 129.14 82.81) (end 129.46 82.81) (width 0.5) (layer B.Cu) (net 4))
 (segment (start 125.39 79.06) (end 129.14 82.81) (width 0.5) (layer B.Cu) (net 4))
 (via (at 129.46 82.81) (size 0.8) (drill 0.4) (layers F.Cu B.Cu) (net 4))
 (segment (start 124.64 79.06) (end 125.39 79.06) (width 0.5) (layer B.Cu) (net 4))
 (segment (start 136.18 82.81) (end 136.34 82.97) (width 0.5) (layer F.Cu) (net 4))
 (segment (start 129.46 82.81) (end 136.18 82.81) (width 0.5) (layer F.Cu) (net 4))
 (segment (start 139.7 67.28) (end 139.75 67.33) (width 0.5) (layer F.Cu) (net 5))
 (segment (start 134.83 67.28) (end 139.7 67.28) (width 0.5) (layer F.Cu) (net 5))
 (via (at 144.77 81.29) (size 0.8) (drill 0.4) (layers F.Cu B.Cu) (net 5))
 (segment (start 143.09 82.97) (end 144.77 81.29) (width 0.5) (layer F.Cu) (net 5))
 (segment (start 140.34 82.97) (end 143.09 82.97) (width 0.5) (layer F.Cu) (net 5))
 (via (at 144.81 71.96) (size 0.8) (drill 0.4) (layers F.Cu B.Cu) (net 5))
 (segment (start 144.77 72) (end 144.81 71.96) (width 0.5) (layer B.Cu) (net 5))
 (segment (start 144.77 81.29) (end 144.77 72) (width 0.5) (layer B.Cu) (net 5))
 (segment (start 140.745685 67.33) (end 140.55 67.33) (width 0.5) (layer F.Cu) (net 5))
 (segment (start 144.81 71.394315) (end 140.745685 67.33) (width 0.5) (layer F.Cu) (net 5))
 (segment (start 140.55 67.33) (end 139.75 67.33) (width 0.5) (layer F.Cu) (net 5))
 (segment (start 144.81 71.96) (end 144.81 71.394315) (width 0.5) (layer F.Cu) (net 5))
 (segment (start 138.73 69.6) (end 138.09 68.96) (width 0.5) (layer F.Cu) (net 6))
 (segment (start 138.73 71.1) (end 138.73 69.6) (width 0.5) (layer F.Cu) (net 6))
 (segment (start 132.51 68.96) (end 130.83 67.28) (width 0.5) (layer F.Cu) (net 6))
 (segment (start 138.09 68.96) (end 132.51 68.96) (width 0.5) (layer F.Cu) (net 6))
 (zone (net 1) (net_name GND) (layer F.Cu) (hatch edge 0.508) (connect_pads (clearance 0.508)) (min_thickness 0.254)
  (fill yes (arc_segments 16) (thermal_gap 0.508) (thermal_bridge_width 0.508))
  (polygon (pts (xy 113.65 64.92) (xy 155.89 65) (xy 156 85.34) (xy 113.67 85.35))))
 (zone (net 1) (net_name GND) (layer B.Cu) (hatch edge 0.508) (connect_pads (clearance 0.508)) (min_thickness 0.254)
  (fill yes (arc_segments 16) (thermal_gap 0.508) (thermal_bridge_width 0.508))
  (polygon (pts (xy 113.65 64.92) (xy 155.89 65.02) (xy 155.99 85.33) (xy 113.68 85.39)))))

